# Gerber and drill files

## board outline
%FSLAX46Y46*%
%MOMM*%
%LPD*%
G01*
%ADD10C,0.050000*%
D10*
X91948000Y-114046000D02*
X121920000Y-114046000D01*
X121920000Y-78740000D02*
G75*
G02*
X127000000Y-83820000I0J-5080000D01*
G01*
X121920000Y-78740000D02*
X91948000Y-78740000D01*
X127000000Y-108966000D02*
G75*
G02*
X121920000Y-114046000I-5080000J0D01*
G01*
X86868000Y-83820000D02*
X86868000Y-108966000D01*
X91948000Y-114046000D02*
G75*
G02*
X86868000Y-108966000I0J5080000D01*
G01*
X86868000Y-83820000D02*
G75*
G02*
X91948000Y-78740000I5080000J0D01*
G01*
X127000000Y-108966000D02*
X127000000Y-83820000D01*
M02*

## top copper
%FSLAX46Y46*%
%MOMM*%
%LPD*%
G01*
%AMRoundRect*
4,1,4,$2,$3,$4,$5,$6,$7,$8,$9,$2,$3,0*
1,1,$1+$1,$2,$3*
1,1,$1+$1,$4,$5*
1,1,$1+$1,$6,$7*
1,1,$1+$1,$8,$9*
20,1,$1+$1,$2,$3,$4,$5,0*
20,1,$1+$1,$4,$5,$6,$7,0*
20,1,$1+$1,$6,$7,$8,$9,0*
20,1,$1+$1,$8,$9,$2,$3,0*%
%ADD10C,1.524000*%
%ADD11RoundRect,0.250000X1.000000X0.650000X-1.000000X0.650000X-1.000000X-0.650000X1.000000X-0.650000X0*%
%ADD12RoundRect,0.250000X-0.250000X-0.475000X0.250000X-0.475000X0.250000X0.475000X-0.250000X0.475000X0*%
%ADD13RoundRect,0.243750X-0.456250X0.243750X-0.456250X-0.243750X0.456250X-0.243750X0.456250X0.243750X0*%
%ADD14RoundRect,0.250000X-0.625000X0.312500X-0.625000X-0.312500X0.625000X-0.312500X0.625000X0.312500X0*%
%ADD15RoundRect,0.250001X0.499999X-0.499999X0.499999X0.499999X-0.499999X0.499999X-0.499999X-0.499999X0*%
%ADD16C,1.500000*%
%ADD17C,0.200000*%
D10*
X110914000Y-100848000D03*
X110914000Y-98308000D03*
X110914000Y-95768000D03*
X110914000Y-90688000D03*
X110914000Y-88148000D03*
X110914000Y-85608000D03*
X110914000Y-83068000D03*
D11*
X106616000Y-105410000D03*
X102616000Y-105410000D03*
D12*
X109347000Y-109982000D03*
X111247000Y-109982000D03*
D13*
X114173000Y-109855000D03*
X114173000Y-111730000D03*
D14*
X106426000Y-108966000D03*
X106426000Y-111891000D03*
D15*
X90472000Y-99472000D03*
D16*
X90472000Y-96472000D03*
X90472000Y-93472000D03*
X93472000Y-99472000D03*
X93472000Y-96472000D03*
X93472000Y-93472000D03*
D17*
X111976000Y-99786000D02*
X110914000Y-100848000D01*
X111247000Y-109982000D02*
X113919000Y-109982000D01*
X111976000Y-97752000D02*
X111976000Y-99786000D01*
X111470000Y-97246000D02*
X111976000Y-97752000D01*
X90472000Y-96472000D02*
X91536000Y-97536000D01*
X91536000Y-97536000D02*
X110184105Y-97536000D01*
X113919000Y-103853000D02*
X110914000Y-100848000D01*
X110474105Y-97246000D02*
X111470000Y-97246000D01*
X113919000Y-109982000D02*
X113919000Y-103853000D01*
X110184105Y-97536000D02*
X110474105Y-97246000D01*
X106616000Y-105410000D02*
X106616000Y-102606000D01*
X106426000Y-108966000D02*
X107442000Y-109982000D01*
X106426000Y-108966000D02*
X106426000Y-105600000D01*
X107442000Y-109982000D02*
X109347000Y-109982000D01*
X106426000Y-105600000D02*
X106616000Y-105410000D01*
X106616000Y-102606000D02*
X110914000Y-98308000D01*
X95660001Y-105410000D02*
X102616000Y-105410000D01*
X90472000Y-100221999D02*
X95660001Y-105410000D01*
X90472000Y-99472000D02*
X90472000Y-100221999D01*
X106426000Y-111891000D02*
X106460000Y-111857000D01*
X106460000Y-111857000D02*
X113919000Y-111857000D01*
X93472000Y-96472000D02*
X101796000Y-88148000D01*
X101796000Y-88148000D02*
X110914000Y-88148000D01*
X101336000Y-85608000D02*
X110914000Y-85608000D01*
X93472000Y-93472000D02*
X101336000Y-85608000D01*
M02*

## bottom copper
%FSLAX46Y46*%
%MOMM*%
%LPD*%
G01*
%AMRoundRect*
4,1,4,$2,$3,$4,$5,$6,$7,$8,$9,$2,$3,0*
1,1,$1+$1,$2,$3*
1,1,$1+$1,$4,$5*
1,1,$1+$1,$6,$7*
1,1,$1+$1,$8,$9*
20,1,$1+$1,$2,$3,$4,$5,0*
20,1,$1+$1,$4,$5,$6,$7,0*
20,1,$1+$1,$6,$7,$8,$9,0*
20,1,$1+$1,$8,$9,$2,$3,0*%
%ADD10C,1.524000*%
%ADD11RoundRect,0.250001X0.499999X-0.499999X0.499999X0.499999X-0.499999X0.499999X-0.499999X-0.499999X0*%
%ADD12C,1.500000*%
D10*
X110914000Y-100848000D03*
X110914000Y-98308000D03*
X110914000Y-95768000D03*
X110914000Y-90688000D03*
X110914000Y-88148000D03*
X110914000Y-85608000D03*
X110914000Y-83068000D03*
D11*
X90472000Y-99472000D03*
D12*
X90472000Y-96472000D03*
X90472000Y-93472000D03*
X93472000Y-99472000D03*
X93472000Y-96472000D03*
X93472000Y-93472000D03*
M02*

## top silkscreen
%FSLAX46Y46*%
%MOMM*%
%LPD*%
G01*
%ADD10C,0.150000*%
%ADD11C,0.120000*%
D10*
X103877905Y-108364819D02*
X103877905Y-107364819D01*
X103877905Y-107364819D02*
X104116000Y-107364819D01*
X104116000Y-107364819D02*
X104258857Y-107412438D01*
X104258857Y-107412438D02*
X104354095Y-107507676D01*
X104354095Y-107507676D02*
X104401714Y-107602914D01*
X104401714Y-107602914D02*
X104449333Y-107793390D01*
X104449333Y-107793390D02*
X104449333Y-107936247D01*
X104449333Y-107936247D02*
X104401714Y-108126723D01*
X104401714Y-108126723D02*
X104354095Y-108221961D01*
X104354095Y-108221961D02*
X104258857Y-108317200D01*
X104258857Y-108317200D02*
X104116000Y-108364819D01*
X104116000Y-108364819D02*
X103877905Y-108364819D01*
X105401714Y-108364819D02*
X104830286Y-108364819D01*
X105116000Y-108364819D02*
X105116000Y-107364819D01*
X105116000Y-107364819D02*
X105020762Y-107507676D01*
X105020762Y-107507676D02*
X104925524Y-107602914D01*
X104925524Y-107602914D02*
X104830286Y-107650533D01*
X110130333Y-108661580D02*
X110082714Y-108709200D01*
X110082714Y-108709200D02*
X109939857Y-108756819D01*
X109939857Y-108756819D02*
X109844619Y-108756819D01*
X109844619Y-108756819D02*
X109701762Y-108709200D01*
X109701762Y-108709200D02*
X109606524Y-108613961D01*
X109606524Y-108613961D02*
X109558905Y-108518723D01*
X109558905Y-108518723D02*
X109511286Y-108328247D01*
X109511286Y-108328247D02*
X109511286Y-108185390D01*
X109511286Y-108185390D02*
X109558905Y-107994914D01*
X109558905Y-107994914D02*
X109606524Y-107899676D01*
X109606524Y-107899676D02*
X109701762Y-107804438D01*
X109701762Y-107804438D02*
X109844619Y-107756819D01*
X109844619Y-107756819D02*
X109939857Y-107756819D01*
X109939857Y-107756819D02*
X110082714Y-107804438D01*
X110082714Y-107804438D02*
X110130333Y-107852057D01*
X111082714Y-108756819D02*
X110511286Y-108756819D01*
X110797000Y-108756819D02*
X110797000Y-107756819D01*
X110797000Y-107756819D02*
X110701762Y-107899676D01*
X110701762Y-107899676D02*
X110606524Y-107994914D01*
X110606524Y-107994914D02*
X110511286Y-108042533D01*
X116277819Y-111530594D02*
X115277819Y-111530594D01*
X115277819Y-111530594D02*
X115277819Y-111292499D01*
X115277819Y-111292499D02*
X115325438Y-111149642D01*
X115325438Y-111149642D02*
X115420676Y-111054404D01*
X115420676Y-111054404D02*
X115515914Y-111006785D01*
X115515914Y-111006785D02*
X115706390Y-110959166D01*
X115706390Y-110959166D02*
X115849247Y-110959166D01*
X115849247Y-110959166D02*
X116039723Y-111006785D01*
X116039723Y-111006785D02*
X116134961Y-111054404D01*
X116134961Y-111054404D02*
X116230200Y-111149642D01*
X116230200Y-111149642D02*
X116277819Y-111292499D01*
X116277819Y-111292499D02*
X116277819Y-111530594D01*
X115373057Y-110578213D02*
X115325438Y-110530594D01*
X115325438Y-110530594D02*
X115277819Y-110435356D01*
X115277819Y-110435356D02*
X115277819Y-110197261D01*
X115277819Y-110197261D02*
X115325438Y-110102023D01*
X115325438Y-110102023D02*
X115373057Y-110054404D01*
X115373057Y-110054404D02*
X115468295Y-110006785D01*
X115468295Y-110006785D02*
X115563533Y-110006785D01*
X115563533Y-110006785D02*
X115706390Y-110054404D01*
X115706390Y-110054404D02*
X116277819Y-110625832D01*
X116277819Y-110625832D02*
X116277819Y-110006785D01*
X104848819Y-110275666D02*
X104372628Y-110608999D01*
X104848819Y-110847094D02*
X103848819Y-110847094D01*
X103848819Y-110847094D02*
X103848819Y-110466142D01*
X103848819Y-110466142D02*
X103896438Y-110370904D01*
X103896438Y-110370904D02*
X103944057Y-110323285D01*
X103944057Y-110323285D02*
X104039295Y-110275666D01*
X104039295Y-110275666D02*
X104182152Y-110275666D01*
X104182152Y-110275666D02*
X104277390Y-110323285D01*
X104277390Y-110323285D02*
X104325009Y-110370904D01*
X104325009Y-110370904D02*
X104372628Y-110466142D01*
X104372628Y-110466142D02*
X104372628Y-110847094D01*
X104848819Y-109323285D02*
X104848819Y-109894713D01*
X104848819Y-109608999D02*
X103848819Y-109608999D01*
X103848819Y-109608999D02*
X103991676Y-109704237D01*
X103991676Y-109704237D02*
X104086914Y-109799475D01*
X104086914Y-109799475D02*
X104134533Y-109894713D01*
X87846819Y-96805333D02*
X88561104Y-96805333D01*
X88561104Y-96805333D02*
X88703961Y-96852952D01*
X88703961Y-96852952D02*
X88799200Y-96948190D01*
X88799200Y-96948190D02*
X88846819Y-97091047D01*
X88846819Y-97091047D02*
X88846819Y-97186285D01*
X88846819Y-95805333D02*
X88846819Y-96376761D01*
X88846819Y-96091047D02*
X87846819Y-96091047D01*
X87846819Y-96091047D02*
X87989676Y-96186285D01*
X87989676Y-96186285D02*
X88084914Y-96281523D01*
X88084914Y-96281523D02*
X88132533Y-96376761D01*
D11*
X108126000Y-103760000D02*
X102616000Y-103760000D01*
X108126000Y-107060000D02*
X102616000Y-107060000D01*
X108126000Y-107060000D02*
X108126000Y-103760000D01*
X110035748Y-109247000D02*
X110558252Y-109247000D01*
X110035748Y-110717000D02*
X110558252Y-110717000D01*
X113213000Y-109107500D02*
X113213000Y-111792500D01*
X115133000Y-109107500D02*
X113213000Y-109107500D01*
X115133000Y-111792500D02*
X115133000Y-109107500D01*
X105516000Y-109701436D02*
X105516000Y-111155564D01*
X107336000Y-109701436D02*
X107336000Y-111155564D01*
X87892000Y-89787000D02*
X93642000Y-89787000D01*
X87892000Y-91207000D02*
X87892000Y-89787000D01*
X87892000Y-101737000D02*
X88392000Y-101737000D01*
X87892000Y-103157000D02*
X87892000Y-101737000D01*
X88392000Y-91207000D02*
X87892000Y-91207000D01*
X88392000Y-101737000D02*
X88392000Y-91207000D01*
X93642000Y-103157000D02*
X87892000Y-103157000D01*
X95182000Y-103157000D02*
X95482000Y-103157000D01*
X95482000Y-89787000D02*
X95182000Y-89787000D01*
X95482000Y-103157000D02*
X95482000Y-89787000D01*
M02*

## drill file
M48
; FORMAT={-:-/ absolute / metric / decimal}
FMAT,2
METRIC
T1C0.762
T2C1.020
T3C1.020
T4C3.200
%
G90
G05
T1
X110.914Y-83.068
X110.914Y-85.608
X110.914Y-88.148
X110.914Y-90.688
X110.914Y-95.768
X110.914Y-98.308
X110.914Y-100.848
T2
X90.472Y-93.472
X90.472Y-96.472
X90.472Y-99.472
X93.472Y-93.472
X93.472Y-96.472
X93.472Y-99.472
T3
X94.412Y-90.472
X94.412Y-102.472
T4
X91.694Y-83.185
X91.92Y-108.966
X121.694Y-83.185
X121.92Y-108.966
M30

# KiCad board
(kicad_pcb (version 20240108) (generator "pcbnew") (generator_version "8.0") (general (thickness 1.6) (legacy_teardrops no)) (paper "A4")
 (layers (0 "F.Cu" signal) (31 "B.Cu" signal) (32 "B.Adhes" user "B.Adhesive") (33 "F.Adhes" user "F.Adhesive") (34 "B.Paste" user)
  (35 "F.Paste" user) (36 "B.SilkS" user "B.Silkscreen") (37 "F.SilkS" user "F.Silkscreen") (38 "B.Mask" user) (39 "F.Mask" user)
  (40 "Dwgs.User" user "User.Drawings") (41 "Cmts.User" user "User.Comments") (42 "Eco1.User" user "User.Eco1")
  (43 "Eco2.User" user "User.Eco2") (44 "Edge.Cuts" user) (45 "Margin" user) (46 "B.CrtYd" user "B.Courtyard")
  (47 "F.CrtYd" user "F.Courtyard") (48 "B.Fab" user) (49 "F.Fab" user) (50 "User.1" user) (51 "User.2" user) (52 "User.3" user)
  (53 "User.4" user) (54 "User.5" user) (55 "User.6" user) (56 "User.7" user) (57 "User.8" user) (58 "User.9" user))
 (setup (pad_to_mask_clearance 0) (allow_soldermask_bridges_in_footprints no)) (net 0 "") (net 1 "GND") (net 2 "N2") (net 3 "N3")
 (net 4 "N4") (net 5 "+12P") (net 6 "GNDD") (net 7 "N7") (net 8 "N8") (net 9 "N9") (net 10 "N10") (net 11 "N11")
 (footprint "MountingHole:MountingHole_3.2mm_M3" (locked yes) (layer "F.Cu") (at 121.694 83.185)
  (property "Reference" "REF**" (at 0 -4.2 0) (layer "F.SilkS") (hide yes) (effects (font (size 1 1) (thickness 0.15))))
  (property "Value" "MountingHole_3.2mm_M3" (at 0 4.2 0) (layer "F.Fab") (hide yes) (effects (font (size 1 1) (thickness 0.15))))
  (pad "" np_thru_hole circle (at 0 0) (size 3.2 3.2) (drill 3.2) (layers "*.Cu" "*.Mask")))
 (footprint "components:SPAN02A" (layer "F.Cu") (at 110.914 100.848 90)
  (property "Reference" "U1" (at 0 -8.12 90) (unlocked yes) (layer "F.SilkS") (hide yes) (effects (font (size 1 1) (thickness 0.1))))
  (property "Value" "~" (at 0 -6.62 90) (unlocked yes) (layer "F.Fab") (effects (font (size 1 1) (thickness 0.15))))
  (pad "1" thru_hole circle (at 0 0 90) (size 1.524 1.524) (drill 0.762) (layers "*.Cu" "*.Mask") (remove_unused_layers no) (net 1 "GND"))
  (pad "2" thru_hole circle (at 2.54 0 90) (size 1.524 1.524) (drill 0.762) (layers "*.Cu" "*.Mask") (remove_unused_layers no) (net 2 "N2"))
  (pad "3" thru_hole circle (at 5.08 0 90) (size 1.524 1.524) (drill 0.762) (layers "*.Cu" "*.Mask") (remove_unused_layers no) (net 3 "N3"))
  (pad "5" thru_hole circle (at 10.16 0 90) (size 1.524 1.524) (drill 0.762) (layers "*.Cu" "*.Mask") (remove_unused_layers no) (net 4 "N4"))
  (pad "6" thru_hole circle (at 12.7 0 90) (size 1.524 1.524) (drill 0.762) (layers "*.Cu" "*.Mask") (remove_unused_layers no)
   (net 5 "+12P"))
  (pad "7" thru_hole circle (at 15.24 0 90) (size 1.524 1.524) (drill 0.762) (layers "*.Cu" "*.Mask") (remove_unused_layers no)
   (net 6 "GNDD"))
  (pad "8" thru_hole circle (at 17.78 0 90) (size 1.524 1.524) (drill 0.762) (layers "*.Cu" "*.Mask") (remove_unused_layers no) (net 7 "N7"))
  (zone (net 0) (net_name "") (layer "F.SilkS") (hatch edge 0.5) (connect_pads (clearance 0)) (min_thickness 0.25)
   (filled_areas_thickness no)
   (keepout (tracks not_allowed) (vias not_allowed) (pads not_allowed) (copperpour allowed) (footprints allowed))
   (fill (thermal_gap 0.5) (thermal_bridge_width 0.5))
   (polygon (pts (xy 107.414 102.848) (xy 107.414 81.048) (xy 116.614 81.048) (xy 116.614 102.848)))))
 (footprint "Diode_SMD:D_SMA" (layer "F.Cu") (at 104.616 105.41 180)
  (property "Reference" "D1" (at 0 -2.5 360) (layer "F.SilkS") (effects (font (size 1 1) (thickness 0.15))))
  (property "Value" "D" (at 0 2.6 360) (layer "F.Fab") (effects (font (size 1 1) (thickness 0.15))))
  (fp_line (start -3.51 1.65) (end 2 1.65) (stroke (width 0.12) (type solid)) (layer "F.SilkS"))
  (fp_line (start -3.51 -1.65) (end 2 -1.65) (stroke (width 0.12) (type solid)) (layer "F.SilkS"))
  (fp_line (start -3.51 -1.65) (end -3.51 1.65) (stroke (width 0.12) (type solid)) (layer "F.SilkS"))
  (pad "1" smd roundrect (at -2 0 180) (size 2.5 1.8) (layers "F.Cu" "F.Paste" "F.Mask") (roundrect_rratio 0.1388888889) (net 2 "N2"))
  (pad "2" smd roundrect (at 2 0 180) (size 2.5 1.8) (layers "F.Cu" "F.Paste" "F.Mask") (roundrect_rratio 0.1388888889) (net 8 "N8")))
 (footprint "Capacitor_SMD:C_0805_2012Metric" (layer "F.Cu") (at 110.297 109.982)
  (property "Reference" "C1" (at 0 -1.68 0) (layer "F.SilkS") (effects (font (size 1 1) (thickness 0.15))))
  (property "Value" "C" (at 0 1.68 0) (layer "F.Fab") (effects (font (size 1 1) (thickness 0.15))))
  (fp_line (start -0.261252 -0.735) (end 0.261252 -0.735) (stroke (width 0.12) (type solid)) (layer "F.SilkS"))
  (fp_line (start -0.261252 0.735) (end 0.261252 0.735) (stroke (width 0.12) (type solid)) (layer "F.SilkS"))
  (pad "1" smd roundrect (at -0.95 0) (size 1 1.45) (layers "F.Cu" "F.Paste" "F.Mask") (roundrect_rratio 0.25) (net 2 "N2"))
  (pad "2" smd roundrect (at 0.95 0) (size 1 1.45) (layers "F.Cu" "F.Paste" "F.Mask") (roundrect_rratio 0.25) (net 1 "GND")))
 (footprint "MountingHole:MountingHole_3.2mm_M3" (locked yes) (layer "F.Cu") (at 91.694 83.185)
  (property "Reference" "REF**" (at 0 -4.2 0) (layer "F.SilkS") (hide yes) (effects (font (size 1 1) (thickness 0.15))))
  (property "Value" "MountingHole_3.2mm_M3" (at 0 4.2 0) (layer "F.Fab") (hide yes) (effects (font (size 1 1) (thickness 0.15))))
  (pad "" np_thru_hole circle (at 0 0) (size 3.2 3.2) (drill 3.2) (layers "*.Cu" "*.Mask")))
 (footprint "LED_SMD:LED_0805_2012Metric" (layer "F.Cu") (at 114.173 110.7925 -90)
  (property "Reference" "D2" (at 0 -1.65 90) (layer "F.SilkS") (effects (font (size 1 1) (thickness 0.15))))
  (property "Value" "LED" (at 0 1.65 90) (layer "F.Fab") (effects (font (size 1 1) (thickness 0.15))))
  (fp_line (start -1.685 0.96) (end 1 0.96) (stroke (width 0.12) (type solid)) (layer "F.SilkS"))
  (fp_line (start -1.685 -0.96) (end -1.685 0.96) (stroke (width 0.12) (type solid)) (layer "F.SilkS"))
  (fp_line (start 1 -0.96) (end -1.685 -0.96) (stroke (width 0.12) (type solid)) (layer "F.SilkS"))
  (pad "1" smd roundrect (at -0.9375 0 270) (size 0.975 1.4) (layers "F.Cu" "F.Paste" "F.Mask") (roundrect_rratio 0.25) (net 1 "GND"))
  (pad "2" smd roundrect (at 0.9375 0 270) (size 0.975 1.4) (layers "F.Cu" "F.Paste" "F.Mask") (roundrect_rratio 0.25) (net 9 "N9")))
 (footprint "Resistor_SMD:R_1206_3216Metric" (layer "F.Cu") (at 106.426 110.4285 -90)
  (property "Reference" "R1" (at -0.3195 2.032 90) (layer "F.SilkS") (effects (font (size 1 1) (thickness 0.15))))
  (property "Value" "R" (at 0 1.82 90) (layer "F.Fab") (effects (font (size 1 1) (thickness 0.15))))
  (fp_line (start -0.727064 0.91) (end 0.727064 0.91) (stroke (width 0.12) (type solid)) (layer "F.SilkS"))
  (fp_line (start -0.727064 -0.91) (end 0.727064 -0.91) (stroke (width 0.12) (type solid)) (layer "F.SilkS"))
  (pad "1" smd roundrect (at -1.4625 0 270) (size 1.125 1.75) (layers "F.Cu" "F.Paste" "F.Mask") (roundrect_rratio 0.222222) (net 2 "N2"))
  (pad "2" smd roundrect (at 1.4625 0 270) (size 1.125 1.75) (layers "F.Cu" "F.Paste" "F.Mask") (roundrect_rratio 0.222222) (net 9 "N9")))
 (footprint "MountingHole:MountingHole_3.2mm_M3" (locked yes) (layer "F.Cu") (at 91.92 108.966)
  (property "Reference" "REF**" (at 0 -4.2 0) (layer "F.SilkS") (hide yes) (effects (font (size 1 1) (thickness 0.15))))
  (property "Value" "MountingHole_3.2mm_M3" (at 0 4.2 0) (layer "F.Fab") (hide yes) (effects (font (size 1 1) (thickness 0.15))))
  (pad "" np_thru_hole circle (at 0 0) (size 3.2 3.2) (drill 3.2) (layers "*.Cu" "*.Mask")))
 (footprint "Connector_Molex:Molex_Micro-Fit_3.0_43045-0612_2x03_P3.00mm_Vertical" (layer "F.Cu") (at 90.472 99.472 90)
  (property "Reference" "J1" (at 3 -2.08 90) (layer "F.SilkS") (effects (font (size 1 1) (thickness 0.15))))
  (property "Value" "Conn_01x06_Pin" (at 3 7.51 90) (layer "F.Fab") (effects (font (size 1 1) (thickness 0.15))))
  (fp_line (start 9.685 -2.58) (end 9.685 3.17) (stroke (width 0.12) (type solid)) (layer "F.SilkS"))
  (fp_line (start 8.265 -2.58) (end 9.685 -2.58) (stroke (width 0.12) (type solid)) (layer "F.SilkS"))
  (fp_line (start -2.265 -2.58) (end -2.265 -2.08) (stroke (width 0.12) (type solid)) (layer "F.SilkS"))
  (fp_line (start -3.685 -2.58) (end -2.265 -2.58) (stroke (width 0.12) (type solid)) (layer "F.SilkS"))
  (fp_line (start 8.265 -2.08) (end 8.265 -2.58) (stroke (width 0.12) (type solid)) (layer "F.SilkS"))
  (fp_line (start -2.265 -2.08) (end 8.265 -2.08) (stroke (width 0.12) (type solid)) (layer "F.SilkS"))
  (fp_line (start -3.685 3.17) (end -3.685 -2.58) (stroke (width 0.12) (type solid)) (layer "F.SilkS"))
  (fp_line (start -3.685 4.71) (end -3.685 5.01) (stroke (width 0.12) (type solid)) (layer "F.SilkS"))
  (fp_line (start 9.685 5.01) (end 9.685 4.71) (stroke (width 0.12) (type solid)) (layer "F.SilkS"))
  (fp_line (start -3.685 5.01) (end 9.685 5.01) (stroke (width 0.12) (type solid)) (layer "F.SilkS"))
  (pad "" np_thru_hole circle (at -3 3.94 90) (size 1.02 1.02) (drill 1.02) (layers "*.Cu" "*.Mask"))
  (pad "" np_thru_hole circle (at 9 3.94 90) (size 1.02 1.02) (drill 1.02) (layers "*.Cu" "*.Mask"))
  (pad "1" thru_hole roundrect (at 0 0 90) (size 1.5 1.5) (drill 1.02) (layers "*.Cu" "*.Mask") (remove_unused_layers no)
   (roundrect_rratio 0.166667) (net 8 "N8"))
  (pad "2" thru_hole circle (at 3 0 90) (size 1.5 1.5) (drill 1.02) (layers "*.Cu" "*.Mask") (remove_unused_layers no) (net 1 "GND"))
  (pad "3" thru_hole circle (at 6 0 90) (size 1.5 1.5) (drill 1.02) (layers "*.Cu" "*.Mask") (remove_unused_layers no) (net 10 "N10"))
  (pad "4" thru_hole circle (at 0 3 90) (size 1.5 1.5) (drill 1.02) (layers "*.Cu" "*.Mask") (remove_unused_layers no) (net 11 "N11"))
  (pad "5" thru_hole circle (at 3 3 90) (size 1.5 1.5) (drill 1.02) (layers "*.Cu" "*.Mask") (remove_unused_layers no) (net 5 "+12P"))
  (pad "6" thru_hole circle (at 6 3 90) (size 1.5 1.5) (drill 1.02) (layers "*.Cu" "*.Mask") (remove_unused_layers no) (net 6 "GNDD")))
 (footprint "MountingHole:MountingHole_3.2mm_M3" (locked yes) (layer "F.Cu") (at 121.92 108.966)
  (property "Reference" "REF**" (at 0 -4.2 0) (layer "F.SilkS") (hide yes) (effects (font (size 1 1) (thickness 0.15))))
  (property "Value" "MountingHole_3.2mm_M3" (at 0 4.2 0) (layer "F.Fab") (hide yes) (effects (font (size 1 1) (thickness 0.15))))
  (pad "" np_thru_hole circle (at 0 0) (size 3.2 3.2) (drill 3.2) (layers "*.Cu" "*.Mask")))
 (gr_line (start 91.948 114.046) (end 121.92 114.046) (stroke (width 0.05) (type default)) (layer "Edge.Cuts"))
 (gr_arc (start 121.92 78.74) (mid 125.512102 80.227898) (end 127 83.82) (stroke (width 0.05) (type default)) (layer "Edge.Cuts"))
 (gr_line (start 121.92 78.74) (end 91.948 78.74) (stroke (width 0.05) (type default)) (layer "Edge.Cuts"))
 (gr_arc (start 127 108.966) (mid 125.512102 112.558102) (end 121.92 114.046) (stroke (width 0.05) (type default)) (layer "Edge.Cuts"))
 (gr_line (start 86.868 83.82) (end 86.868 108.966) (stroke (width 0.05) (type default)) (layer "Edge.Cuts"))
 (gr_arc (start 91.948 114.046) (mid 88.355898 112.558102) (end 86.868 108.966) (stroke (width 0.05) (type default)) (layer "Edge.Cuts"))
 (gr_arc (start 86.868 83.82) (mid 88.355898 80.227898) (end 91.948 78.74) (stroke (width 0.05) (type default)) (layer "Edge.Cuts"))
 (gr_line (start 127 108.966) (end 127 83.82) (stroke (width 0.05) (type default)) (layer "Edge.Cuts"))
 (segment (start 111.976 99.786) (end 110.914 100.848) (width 0.2) (layer "F.Cu") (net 1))
 (segment (start 111.247 109.982) (end 113.919 109.982) (width 0.2) (layer "F.Cu") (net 1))
 (segment (start 111.976 97.752) (end 111.976 99.786) (width 0.2) (layer "F.Cu") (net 1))
 (segment (start 111.47 97.246) (end 111.976 97.752) (width 0.2) (layer "F.Cu") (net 1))
 (segment (start 90.472 96.472) (end 91.536 97.536) (width 0.2) (layer "F.Cu") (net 1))
 (segment (start 91.536 97.536) (end 110.184105 97.536) (width 0.2) (layer "F.Cu") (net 1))
 (segment (start 113.919 103.853) (end 110.914 100.848) (width 0.2) (layer "F.Cu") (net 1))
 (segment (start 110.474105 97.246) (end 111.47 97.246) (width 0.2) (layer "F.Cu") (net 1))
 (segment (start 113.919 109.982) (end 113.919 103.853) (width 0.2) (layer "F.Cu") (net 1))
 (segment (start 110.184105 97.536) (end 110.474105 97.246) (width 0.2) (layer "F.Cu") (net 1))
 (segment (start 106.616 105.41) (end 106.616 102.606) (width 0.2) (layer "F.Cu") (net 2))
 (segment (start 106.426 108.966) (end 107.442 109.982) (width 0.2) (layer "F.Cu") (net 2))
 (segment (start 106.426 108.966) (end 106.426 105.6) (width 0.2) (layer "F.Cu") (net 2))
 (segment (start 107.442 109.982) (end 109.347 109.982) (width 0.2) (layer "F.Cu") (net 2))
 (segment (start 106.426 105.6) (end 106.616 105.41) (width 0.2) (layer "F.Cu") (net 2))
 (segment (start 106.616 102.606) (end 110.914 98.308) (width 0.2) (layer "F.Cu") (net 2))
 (segment (start 95.660001 105.41) (end 102.616 105.41) (width 0.2) (layer "F.Cu") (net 8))
 (segment (start 90.472 100.221999) (end 95.660001 105.41) (width 0.2) (layer "F.Cu") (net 8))
 (segment (start 90.472 99.472) (end 90.472 100.221999) (width 0.2) (layer "F.Cu") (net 8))
 (segment (start 106.426 111.891) (end 106.46 111.857) (width 0.2) (layer "F.Cu") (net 9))
 (segment (start 106.46 111.857) (end 113.919 111.857) (width 0.2) (layer "F.Cu") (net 9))
 (segment (start 93.472 96.472) (end 101.796 88.148) (width 0.2) (layer "F.Cu") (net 5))
 (segment (start 101.796 88.148) (end 110.914 88.148) (width 0.2) (layer "F.Cu") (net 5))
 (segment (start 101.336 85.608) (end 110.914 85.608) (width 0.2) (layer "F.Cu") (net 6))
 (segment (start 93.472 93.472) (end 101.336 85.608) (width 0.2) (layer "F.Cu") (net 6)))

